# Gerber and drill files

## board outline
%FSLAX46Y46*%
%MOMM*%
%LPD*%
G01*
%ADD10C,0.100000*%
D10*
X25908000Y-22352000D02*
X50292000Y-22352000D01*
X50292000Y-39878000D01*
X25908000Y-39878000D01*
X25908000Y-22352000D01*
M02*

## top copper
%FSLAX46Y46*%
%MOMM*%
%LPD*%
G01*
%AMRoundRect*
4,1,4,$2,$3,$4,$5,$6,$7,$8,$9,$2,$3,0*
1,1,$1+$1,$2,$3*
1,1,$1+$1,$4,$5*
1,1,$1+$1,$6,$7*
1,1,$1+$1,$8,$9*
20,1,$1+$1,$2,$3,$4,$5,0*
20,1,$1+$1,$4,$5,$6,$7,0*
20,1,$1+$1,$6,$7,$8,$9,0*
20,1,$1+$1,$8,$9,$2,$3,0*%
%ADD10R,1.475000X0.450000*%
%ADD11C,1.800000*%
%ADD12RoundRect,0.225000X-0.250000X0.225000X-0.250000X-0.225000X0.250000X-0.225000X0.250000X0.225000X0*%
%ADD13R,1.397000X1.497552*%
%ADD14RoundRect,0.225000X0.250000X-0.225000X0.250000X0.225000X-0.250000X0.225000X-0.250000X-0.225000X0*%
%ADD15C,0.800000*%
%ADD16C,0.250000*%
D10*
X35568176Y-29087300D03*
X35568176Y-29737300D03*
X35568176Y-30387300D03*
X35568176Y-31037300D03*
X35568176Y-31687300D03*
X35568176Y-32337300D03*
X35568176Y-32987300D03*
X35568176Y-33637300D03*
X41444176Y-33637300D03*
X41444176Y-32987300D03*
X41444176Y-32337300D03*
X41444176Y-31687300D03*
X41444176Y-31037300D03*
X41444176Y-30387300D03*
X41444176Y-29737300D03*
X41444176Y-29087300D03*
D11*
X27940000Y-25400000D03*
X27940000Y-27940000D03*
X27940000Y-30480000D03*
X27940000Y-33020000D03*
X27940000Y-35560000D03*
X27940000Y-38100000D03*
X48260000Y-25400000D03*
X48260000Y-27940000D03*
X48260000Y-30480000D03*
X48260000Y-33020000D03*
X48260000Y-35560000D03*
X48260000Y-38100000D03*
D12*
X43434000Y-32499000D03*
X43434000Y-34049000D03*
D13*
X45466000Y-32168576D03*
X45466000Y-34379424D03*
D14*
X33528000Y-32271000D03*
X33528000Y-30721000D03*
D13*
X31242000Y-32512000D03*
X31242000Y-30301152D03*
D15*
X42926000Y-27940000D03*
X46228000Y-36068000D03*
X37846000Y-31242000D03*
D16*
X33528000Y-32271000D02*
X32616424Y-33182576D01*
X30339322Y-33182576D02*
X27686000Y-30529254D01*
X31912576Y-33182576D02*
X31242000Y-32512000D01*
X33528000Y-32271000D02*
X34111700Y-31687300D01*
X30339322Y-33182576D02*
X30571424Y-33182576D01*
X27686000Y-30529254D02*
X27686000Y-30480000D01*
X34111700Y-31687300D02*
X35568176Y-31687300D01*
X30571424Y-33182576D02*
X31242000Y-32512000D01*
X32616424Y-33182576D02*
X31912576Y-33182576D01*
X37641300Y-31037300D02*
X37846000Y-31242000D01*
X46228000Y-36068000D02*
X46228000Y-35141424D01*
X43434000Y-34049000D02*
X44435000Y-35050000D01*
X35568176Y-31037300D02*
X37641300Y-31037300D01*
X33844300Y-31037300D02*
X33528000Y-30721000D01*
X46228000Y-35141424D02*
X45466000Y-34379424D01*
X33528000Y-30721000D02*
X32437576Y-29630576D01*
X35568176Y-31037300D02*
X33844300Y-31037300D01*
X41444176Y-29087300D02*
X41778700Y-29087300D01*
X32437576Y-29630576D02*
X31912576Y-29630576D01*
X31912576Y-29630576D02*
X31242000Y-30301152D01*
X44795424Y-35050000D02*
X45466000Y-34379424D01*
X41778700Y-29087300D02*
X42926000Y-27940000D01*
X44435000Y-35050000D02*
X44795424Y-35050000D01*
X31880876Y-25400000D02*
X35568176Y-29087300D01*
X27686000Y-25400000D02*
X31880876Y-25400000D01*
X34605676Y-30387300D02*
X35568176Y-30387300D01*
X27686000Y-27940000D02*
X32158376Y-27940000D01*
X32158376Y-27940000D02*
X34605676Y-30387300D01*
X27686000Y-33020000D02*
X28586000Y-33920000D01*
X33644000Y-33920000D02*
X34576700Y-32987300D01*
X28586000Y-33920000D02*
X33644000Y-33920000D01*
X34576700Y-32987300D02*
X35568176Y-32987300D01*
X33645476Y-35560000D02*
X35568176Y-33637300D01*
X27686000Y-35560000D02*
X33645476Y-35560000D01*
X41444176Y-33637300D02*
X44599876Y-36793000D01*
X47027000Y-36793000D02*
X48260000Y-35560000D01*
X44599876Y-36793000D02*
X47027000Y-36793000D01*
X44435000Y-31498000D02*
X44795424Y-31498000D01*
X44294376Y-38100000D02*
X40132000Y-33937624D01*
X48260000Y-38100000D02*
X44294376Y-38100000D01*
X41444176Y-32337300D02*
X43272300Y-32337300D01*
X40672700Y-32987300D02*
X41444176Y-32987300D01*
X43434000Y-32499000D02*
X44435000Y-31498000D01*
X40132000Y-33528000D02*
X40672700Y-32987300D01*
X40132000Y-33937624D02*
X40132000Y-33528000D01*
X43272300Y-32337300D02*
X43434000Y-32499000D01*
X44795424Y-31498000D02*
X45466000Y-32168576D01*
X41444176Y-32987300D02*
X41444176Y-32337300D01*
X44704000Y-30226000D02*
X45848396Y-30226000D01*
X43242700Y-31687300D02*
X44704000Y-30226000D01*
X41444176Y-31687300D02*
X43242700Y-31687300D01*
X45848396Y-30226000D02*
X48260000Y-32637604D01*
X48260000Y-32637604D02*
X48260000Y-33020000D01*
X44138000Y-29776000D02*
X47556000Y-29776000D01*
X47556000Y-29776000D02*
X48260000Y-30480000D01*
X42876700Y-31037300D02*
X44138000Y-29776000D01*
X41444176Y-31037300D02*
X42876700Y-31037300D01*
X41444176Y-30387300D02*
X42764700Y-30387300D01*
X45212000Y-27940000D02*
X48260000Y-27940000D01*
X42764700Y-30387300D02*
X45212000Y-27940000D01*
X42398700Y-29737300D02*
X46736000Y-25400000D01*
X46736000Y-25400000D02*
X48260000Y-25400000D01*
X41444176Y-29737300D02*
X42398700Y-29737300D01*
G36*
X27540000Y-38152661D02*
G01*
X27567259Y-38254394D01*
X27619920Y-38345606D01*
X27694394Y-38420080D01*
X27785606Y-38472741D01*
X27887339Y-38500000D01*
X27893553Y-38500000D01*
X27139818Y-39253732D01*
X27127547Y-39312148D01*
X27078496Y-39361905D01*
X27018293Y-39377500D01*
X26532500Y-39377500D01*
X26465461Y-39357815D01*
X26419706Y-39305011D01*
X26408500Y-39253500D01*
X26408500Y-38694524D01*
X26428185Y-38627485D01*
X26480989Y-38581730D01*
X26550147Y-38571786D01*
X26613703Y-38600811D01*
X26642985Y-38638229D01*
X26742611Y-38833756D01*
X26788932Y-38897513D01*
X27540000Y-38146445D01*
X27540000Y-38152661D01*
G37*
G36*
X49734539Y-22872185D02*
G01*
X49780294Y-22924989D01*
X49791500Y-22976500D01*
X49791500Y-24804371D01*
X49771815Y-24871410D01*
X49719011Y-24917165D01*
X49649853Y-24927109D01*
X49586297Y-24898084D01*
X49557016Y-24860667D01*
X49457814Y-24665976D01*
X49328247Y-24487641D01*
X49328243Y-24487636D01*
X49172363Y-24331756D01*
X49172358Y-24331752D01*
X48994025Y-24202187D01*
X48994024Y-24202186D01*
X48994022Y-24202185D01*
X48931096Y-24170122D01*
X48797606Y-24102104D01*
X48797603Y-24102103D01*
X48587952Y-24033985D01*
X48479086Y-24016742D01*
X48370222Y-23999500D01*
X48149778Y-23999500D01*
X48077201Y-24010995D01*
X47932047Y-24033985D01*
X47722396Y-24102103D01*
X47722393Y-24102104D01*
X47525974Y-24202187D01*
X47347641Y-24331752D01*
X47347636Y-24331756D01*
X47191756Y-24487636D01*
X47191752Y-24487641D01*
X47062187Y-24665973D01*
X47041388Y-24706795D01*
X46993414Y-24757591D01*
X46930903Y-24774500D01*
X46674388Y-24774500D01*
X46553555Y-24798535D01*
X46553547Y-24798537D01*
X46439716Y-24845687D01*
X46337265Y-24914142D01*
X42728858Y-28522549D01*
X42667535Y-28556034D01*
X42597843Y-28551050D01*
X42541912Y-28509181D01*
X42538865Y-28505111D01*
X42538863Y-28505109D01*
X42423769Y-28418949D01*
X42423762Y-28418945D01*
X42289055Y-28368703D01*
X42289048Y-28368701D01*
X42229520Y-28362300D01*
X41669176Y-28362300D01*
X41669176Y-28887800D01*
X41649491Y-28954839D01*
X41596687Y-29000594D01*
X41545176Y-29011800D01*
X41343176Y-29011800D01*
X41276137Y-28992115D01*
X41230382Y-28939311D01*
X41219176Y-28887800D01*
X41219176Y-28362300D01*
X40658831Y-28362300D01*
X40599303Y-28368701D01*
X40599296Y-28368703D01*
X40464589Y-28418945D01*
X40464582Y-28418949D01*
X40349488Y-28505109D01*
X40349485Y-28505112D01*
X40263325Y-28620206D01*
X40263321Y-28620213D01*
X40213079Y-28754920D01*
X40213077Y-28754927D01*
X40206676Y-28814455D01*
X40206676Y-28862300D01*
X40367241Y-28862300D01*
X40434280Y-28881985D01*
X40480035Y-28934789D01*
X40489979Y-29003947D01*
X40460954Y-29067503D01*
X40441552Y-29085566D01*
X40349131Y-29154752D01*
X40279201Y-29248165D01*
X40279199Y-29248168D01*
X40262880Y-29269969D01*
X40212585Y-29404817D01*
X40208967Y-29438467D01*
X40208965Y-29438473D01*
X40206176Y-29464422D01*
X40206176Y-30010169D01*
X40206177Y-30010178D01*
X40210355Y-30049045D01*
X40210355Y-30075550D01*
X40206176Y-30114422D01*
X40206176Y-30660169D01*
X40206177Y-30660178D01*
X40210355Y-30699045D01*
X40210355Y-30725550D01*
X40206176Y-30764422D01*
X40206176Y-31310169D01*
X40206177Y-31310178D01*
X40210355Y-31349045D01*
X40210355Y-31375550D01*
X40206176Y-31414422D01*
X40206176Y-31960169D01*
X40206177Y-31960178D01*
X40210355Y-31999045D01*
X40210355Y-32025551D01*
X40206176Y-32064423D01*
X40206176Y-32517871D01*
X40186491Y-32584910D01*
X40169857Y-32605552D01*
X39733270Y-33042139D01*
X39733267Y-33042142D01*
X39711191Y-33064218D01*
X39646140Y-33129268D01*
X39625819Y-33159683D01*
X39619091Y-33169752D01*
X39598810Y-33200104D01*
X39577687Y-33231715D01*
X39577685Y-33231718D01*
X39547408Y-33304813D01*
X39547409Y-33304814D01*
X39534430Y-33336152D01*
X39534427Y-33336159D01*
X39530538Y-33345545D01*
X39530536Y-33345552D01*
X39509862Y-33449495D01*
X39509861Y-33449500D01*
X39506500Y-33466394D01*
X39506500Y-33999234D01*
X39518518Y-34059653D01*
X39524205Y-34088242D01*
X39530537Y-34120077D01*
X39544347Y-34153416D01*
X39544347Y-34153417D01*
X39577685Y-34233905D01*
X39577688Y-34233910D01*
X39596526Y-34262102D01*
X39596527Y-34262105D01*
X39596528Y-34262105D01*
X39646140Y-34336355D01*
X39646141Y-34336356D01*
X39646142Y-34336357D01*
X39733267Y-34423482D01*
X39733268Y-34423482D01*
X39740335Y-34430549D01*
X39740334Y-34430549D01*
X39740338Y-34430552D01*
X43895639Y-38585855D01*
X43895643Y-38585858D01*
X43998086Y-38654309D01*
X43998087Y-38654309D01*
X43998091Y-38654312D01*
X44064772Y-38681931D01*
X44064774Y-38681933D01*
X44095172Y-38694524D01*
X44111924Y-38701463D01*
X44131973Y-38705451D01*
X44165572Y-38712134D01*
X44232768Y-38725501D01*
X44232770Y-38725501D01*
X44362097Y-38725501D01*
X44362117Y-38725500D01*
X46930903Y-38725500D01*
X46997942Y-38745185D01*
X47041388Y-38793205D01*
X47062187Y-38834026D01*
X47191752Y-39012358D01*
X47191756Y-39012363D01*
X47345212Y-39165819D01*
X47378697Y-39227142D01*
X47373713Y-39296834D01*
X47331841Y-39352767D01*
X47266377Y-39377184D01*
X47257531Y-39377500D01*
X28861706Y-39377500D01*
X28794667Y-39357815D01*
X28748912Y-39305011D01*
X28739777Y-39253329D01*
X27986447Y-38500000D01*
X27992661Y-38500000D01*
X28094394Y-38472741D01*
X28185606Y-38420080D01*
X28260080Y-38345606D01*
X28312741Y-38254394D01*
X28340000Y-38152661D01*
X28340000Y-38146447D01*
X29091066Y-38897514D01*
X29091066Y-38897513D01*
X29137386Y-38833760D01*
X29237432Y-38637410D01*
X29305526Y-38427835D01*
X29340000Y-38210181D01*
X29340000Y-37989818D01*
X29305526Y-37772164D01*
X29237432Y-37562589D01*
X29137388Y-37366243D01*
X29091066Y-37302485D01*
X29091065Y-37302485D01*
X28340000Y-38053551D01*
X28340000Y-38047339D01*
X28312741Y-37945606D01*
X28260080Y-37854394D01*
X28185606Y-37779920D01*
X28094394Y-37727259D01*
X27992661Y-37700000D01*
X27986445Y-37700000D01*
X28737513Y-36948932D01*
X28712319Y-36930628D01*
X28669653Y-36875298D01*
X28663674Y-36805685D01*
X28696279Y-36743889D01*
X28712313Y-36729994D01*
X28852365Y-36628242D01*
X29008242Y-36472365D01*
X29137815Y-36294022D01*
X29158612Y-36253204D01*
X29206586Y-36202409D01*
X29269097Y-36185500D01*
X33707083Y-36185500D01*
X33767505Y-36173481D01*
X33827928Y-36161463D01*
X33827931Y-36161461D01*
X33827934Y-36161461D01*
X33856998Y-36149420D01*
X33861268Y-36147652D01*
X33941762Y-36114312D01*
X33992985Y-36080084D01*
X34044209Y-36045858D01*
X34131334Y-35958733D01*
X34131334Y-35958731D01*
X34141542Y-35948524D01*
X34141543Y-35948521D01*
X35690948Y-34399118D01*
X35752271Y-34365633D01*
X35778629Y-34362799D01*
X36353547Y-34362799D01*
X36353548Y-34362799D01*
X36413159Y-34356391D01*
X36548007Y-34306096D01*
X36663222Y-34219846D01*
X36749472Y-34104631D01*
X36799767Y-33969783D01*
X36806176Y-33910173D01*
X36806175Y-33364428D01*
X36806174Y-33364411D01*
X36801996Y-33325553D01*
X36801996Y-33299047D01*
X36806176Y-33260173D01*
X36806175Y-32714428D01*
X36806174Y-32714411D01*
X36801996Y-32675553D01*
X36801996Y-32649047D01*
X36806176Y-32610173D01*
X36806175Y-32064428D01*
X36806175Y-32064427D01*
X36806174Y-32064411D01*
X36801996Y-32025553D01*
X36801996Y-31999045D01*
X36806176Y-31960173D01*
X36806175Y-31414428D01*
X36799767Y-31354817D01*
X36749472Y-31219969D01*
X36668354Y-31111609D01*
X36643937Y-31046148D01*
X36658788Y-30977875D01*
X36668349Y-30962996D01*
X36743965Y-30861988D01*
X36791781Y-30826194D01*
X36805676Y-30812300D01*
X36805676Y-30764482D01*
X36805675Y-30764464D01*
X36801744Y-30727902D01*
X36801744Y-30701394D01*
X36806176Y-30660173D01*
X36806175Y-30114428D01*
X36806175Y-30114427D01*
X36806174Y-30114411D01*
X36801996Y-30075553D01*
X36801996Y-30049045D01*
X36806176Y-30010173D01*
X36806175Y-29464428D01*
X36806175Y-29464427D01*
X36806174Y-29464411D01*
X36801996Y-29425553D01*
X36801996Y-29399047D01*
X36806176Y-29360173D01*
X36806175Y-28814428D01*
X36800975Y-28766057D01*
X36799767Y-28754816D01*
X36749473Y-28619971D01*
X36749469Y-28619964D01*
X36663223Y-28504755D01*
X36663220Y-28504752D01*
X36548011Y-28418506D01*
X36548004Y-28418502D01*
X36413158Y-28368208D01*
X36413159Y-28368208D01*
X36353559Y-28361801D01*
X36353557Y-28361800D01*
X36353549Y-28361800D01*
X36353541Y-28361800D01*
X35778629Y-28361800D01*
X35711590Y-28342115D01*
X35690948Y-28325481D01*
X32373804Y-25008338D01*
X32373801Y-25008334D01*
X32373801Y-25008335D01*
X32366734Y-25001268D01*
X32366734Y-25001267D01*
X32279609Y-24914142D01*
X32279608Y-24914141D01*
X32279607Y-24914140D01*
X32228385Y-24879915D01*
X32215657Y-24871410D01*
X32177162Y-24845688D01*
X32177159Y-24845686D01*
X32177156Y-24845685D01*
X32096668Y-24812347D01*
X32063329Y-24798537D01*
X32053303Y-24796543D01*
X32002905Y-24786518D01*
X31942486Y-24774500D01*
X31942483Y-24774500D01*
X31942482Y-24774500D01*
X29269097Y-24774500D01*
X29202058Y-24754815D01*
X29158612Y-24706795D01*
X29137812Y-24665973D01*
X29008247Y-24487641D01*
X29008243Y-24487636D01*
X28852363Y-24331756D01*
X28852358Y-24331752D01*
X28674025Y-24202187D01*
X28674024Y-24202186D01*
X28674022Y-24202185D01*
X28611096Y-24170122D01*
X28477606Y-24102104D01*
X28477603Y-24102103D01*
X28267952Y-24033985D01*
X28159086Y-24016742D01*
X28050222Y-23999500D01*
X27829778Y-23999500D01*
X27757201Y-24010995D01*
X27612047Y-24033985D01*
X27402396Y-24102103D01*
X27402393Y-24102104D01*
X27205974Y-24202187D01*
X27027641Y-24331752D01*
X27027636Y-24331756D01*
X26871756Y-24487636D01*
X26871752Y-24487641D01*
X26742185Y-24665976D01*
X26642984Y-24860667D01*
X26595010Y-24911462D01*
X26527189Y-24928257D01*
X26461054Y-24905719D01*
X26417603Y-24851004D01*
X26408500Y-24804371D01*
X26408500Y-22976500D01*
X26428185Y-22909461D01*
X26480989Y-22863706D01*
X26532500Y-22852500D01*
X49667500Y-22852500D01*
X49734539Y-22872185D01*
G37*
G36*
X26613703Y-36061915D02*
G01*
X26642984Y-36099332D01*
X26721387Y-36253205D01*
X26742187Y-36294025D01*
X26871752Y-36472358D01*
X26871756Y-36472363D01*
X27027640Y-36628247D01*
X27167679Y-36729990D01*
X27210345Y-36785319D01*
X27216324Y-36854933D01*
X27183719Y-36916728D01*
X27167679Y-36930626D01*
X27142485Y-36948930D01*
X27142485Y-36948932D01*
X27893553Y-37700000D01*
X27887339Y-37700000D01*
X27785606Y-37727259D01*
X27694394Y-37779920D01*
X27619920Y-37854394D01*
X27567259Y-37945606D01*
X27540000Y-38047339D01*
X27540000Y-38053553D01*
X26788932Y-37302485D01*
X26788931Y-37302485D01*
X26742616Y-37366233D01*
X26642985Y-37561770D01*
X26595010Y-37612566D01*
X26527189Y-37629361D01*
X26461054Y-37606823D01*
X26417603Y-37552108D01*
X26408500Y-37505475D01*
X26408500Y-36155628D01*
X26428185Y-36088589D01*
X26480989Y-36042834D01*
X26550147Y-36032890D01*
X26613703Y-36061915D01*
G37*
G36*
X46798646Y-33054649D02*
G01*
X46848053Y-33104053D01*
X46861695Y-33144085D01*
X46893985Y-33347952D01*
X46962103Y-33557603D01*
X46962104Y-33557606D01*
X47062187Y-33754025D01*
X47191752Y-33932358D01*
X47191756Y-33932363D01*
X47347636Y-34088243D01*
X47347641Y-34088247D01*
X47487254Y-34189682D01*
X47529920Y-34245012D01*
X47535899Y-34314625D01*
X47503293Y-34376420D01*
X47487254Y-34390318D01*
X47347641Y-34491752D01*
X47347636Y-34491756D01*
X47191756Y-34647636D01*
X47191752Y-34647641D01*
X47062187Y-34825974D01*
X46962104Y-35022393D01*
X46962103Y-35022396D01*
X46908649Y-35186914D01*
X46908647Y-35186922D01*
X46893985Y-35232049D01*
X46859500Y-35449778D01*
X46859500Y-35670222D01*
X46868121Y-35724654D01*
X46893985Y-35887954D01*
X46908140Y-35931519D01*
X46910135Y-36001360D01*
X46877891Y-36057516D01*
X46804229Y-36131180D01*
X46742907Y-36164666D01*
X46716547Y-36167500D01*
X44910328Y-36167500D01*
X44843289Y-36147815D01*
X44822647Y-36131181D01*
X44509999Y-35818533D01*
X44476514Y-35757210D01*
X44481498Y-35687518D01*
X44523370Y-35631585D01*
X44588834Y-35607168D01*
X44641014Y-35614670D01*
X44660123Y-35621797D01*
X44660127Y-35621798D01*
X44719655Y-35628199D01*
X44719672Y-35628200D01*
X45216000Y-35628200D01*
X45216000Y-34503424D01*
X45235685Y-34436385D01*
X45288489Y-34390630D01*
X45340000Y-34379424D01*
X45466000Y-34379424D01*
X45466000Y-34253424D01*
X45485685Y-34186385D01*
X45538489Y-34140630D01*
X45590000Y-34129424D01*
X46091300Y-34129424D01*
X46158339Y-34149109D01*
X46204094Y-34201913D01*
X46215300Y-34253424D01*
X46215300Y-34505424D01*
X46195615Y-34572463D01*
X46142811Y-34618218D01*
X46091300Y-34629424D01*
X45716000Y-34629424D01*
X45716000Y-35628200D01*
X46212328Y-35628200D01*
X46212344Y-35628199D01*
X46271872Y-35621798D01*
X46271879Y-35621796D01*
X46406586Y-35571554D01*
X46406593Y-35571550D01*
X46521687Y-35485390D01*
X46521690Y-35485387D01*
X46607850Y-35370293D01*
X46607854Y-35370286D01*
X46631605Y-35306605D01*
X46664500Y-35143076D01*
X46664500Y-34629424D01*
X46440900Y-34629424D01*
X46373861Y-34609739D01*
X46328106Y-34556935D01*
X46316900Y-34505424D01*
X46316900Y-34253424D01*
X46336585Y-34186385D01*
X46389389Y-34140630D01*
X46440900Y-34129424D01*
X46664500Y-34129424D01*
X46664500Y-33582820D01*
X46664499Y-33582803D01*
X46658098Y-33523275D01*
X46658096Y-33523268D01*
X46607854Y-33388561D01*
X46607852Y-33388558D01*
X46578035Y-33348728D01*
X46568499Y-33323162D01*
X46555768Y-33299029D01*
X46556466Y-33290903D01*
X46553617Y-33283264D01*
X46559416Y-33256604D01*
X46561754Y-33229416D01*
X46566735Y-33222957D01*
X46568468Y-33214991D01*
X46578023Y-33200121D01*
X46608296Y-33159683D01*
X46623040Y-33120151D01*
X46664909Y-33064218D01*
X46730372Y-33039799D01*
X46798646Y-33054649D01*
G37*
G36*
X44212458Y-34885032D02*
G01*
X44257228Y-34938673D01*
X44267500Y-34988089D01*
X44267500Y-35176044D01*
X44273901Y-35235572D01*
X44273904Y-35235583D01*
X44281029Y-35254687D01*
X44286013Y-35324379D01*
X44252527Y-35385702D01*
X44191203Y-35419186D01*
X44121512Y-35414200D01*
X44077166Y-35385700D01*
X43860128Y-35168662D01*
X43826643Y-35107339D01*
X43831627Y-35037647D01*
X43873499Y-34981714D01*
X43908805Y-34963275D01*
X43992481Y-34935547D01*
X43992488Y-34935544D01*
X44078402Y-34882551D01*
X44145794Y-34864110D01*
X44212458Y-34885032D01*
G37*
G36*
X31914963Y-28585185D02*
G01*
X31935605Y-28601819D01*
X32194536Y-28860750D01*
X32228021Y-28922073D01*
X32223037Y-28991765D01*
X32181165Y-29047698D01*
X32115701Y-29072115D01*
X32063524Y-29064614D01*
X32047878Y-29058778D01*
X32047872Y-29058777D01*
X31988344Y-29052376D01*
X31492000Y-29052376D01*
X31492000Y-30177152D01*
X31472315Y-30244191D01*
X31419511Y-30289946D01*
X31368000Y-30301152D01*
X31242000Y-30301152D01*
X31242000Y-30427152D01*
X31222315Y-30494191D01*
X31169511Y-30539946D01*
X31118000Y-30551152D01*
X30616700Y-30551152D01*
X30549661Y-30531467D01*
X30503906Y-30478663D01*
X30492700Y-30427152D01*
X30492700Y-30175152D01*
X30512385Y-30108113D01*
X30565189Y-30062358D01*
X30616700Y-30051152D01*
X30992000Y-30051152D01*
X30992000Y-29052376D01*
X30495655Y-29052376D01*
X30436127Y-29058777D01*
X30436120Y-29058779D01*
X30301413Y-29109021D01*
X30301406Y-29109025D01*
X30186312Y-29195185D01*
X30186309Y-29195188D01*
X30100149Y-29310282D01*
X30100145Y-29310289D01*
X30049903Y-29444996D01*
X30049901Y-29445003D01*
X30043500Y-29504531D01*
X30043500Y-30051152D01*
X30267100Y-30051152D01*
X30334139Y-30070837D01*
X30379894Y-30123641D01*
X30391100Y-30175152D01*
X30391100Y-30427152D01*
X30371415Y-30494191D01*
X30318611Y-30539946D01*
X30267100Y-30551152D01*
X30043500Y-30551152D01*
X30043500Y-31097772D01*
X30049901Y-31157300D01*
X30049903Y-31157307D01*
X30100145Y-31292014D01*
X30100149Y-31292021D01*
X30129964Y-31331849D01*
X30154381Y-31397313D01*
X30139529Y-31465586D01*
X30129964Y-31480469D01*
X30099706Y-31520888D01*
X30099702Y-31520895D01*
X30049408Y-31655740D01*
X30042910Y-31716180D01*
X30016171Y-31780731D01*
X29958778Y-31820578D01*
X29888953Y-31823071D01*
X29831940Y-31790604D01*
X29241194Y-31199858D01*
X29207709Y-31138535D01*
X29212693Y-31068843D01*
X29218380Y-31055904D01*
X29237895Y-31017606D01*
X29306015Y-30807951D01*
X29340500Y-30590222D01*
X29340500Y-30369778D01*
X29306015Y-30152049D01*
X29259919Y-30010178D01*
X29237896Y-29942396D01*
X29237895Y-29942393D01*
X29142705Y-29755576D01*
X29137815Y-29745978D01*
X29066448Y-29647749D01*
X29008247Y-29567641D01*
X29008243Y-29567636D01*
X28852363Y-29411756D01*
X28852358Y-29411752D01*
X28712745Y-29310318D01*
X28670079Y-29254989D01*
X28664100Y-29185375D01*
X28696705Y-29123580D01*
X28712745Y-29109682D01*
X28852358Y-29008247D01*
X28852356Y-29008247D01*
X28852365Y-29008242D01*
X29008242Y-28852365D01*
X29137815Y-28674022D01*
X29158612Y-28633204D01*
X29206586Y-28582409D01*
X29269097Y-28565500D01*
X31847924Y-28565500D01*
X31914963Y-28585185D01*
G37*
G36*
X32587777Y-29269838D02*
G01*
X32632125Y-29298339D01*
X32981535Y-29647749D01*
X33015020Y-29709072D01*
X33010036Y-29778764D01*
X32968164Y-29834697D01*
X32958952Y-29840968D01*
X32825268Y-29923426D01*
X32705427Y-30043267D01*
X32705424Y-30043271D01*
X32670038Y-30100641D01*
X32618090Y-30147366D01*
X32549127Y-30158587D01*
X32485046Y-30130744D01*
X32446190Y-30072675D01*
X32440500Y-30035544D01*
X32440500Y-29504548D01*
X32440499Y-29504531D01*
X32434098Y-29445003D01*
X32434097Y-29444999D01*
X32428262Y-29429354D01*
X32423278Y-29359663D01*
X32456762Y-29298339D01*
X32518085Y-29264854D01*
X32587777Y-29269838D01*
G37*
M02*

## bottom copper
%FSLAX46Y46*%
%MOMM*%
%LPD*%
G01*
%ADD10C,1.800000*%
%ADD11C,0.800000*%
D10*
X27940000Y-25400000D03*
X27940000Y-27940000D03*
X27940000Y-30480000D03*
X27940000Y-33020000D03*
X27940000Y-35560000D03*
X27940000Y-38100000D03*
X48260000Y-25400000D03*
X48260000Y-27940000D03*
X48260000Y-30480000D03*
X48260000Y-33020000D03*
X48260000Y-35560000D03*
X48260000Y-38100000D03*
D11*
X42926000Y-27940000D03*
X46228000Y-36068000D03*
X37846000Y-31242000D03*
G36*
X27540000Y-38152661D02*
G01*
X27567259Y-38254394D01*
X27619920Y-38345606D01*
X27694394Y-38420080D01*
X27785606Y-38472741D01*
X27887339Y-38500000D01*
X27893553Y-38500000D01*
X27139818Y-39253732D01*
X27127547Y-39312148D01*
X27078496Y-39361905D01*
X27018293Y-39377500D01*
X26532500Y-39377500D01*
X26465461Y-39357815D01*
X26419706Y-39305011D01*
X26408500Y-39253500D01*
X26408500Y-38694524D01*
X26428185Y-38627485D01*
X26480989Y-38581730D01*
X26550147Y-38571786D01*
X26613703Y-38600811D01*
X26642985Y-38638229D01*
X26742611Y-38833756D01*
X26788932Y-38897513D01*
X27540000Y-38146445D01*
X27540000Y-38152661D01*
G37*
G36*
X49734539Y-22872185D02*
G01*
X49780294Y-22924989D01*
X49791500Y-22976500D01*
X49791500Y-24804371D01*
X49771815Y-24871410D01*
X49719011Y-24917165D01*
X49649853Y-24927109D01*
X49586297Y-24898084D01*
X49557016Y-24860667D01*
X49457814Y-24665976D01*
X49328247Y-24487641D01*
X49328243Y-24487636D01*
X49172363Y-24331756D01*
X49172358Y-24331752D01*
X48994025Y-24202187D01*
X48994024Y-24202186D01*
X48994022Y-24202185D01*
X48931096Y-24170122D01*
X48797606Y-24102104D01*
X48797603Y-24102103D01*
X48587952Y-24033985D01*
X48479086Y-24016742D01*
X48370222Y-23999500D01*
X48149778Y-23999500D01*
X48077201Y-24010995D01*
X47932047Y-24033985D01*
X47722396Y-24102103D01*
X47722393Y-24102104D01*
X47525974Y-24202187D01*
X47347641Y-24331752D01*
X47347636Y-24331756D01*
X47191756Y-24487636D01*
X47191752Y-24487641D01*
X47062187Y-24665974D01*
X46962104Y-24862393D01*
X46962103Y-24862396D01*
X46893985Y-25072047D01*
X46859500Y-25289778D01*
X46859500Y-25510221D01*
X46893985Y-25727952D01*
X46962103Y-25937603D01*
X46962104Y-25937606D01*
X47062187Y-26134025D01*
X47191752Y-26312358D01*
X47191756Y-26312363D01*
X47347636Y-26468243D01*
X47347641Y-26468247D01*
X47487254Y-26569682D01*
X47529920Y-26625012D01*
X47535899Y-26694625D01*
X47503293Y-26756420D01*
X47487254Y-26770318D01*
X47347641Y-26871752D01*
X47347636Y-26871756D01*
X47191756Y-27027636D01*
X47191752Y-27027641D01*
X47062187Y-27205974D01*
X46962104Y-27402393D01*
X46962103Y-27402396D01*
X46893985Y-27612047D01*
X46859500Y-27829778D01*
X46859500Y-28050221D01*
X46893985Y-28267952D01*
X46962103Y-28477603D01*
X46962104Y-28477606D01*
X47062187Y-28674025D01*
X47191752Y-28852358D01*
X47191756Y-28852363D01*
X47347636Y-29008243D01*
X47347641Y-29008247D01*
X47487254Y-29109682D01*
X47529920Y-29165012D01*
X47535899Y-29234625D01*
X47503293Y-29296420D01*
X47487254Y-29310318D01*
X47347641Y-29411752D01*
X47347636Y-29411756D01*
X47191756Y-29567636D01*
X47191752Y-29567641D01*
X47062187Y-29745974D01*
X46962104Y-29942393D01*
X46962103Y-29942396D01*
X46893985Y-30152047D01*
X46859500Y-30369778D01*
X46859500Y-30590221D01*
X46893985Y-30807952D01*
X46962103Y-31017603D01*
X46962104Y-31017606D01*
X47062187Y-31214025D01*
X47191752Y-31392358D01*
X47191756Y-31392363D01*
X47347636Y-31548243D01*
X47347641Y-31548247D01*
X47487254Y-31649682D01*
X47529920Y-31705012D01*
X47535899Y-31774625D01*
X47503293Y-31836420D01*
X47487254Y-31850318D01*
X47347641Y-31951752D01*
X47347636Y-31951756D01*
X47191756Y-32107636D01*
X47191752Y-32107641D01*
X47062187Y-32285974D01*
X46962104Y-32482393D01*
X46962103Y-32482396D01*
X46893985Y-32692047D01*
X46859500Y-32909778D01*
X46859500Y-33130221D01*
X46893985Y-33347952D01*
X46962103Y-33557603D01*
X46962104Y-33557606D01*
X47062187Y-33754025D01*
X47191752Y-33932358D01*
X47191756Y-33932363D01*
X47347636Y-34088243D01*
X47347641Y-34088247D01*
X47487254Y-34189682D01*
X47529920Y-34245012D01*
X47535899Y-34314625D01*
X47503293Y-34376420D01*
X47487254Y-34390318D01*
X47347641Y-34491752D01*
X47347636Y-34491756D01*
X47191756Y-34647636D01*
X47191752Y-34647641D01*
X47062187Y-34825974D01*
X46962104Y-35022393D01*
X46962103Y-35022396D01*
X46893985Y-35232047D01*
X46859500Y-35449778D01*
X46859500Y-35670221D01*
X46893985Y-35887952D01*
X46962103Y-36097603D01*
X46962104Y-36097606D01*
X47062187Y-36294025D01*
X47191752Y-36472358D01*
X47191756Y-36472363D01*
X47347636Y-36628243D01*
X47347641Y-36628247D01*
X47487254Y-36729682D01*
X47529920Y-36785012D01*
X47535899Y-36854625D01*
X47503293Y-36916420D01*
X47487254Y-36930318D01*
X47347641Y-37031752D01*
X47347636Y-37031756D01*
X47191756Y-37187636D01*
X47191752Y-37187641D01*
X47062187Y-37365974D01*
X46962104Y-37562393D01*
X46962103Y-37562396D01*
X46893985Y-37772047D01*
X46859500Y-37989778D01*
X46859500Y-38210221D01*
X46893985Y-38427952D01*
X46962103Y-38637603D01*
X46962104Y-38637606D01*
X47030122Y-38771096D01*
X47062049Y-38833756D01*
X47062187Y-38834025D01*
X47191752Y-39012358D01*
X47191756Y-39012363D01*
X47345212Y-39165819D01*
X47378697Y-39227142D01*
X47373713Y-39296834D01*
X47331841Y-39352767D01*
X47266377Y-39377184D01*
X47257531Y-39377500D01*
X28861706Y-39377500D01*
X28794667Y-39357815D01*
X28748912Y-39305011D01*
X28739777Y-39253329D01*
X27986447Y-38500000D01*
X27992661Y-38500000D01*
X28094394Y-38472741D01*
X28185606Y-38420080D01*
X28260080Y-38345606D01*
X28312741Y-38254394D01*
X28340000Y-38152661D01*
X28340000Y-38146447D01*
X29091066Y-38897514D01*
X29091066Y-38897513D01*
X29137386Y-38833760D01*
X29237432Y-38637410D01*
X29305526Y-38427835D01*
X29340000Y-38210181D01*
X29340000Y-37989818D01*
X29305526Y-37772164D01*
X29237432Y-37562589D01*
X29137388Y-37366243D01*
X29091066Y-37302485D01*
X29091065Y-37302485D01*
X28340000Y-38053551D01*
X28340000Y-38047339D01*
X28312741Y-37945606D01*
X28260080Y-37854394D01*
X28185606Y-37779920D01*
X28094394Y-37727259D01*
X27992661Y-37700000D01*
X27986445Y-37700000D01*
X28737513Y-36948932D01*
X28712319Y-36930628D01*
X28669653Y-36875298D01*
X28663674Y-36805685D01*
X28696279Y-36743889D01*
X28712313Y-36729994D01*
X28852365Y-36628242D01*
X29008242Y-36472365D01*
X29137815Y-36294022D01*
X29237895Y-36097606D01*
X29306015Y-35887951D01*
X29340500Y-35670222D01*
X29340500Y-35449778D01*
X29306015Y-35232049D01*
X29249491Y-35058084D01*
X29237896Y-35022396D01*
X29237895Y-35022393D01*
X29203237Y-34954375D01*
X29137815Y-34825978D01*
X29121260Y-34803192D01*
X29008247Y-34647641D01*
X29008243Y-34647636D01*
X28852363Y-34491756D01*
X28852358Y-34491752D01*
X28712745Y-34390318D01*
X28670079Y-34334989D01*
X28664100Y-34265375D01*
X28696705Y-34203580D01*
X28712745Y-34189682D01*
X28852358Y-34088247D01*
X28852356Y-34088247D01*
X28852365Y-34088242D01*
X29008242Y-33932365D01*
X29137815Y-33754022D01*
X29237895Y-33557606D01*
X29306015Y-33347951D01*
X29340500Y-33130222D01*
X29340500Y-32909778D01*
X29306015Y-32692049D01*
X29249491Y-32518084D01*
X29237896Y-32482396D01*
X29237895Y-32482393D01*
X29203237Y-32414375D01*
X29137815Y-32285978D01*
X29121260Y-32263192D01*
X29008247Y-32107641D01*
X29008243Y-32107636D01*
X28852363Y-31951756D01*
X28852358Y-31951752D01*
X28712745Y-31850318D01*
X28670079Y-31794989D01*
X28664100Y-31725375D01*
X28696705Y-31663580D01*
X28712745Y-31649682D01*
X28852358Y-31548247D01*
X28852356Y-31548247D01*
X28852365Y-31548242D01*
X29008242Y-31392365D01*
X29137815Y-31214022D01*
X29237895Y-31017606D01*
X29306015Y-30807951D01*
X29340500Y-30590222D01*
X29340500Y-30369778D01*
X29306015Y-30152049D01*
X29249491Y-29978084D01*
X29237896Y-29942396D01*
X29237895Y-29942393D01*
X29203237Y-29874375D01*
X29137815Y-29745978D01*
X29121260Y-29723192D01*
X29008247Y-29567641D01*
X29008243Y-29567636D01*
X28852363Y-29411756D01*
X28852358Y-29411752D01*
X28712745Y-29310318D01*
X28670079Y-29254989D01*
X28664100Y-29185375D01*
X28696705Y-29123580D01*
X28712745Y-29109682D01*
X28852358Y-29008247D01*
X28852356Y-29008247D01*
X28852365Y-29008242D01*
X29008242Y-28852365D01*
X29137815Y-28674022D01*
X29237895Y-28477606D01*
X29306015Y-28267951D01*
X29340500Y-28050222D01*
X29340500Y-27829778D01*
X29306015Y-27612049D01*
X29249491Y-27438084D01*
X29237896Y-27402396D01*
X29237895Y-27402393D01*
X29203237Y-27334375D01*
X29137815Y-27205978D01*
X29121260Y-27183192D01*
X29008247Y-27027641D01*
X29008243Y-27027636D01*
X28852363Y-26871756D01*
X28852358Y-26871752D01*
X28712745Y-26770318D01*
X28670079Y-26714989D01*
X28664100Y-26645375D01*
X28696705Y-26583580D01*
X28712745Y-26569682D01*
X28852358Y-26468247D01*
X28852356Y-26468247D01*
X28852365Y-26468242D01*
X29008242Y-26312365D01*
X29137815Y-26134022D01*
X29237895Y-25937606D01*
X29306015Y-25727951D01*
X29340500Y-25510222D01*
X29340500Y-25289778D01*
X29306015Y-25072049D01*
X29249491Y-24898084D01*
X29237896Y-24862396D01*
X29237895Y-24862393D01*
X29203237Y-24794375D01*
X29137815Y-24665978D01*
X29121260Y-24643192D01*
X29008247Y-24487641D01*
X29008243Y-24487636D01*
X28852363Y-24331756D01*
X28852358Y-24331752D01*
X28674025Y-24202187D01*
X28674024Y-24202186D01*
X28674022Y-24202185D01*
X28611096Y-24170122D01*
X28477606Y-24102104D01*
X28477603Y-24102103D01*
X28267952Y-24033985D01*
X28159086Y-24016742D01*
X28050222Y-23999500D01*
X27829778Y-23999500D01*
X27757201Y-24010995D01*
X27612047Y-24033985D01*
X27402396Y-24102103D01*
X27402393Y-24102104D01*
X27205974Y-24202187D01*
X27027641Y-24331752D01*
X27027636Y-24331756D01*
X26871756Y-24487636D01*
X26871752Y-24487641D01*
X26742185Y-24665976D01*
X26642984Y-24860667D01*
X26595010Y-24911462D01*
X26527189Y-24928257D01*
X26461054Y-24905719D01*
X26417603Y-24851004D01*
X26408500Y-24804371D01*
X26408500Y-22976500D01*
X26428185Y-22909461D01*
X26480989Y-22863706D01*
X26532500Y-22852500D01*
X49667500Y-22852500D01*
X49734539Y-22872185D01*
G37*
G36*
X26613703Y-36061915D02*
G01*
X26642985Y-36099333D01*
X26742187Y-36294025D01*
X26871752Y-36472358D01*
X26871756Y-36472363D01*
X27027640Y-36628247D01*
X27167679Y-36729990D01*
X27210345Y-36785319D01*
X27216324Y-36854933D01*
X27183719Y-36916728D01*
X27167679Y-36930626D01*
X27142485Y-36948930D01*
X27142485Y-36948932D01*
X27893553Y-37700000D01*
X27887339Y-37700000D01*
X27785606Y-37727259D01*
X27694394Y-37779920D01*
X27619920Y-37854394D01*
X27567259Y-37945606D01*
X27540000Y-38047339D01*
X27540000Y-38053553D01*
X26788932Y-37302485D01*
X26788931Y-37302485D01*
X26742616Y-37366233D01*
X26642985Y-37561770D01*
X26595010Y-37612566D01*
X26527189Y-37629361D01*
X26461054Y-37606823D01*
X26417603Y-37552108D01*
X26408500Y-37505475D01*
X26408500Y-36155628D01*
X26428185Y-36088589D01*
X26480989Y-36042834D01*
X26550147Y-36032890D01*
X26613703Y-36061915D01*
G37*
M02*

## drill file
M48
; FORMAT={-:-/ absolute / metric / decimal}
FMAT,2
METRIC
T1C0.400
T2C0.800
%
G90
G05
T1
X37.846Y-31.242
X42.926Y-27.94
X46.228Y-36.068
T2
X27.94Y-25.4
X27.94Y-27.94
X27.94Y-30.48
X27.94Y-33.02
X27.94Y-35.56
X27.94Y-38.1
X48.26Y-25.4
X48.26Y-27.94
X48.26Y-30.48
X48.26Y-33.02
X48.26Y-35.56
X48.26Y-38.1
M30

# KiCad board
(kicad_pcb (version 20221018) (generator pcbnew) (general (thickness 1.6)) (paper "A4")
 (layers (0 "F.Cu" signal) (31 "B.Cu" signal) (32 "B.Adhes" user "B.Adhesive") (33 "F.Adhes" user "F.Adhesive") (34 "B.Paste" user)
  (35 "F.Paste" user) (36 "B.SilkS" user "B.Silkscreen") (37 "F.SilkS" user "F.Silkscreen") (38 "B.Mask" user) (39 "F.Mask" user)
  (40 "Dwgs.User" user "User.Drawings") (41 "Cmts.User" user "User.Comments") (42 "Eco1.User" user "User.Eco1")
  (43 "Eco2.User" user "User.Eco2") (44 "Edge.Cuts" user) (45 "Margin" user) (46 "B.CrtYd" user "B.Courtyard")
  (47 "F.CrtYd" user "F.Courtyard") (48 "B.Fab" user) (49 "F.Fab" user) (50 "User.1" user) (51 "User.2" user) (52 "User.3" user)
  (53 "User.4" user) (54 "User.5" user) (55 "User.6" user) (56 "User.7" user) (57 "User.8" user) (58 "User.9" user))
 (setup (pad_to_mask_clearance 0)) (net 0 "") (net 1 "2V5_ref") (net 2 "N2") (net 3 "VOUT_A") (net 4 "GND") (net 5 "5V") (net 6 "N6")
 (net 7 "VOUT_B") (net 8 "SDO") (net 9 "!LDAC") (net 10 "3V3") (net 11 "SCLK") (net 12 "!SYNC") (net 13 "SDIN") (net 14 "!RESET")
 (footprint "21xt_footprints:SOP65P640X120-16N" (layer "F.Cu") (at 38.506176 31.3623)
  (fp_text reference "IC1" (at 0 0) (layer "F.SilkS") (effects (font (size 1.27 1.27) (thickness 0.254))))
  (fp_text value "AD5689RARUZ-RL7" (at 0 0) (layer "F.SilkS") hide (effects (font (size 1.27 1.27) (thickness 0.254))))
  (pad "1" smd rect (at -2.938 -2.275 90) (size 0.45 1.475) (layers "F.Cu" "F.Paste" "F.Mask") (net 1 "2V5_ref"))
  (pad "2" smd rect (at -2.938 -1.625 90) (size 0.45 1.475) (layers "F.Cu" "F.Paste" "F.Mask") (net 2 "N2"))
  (pad "3" smd rect (at -2.938 -0.975 90) (size 0.45 1.475) (layers "F.Cu" "F.Paste" "F.Mask") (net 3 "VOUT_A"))
  (pad "4" smd rect (at -2.938 -0.325 90) (size 0.45 1.475) (layers "F.Cu" "F.Paste" "F.Mask") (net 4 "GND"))
  (pad "5" smd rect (at -2.938 0.325 90) (size 0.45 1.475) (layers "F.Cu" "F.Paste" "F.Mask") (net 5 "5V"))
  (pad "6" smd rect (at -2.938 0.975 90) (size 0.45 1.475) (layers "F.Cu" "F.Paste" "F.Mask") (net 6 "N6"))
  (pad "7" smd rect (at -2.938 1.625 90) (size 0.45 1.475) (layers "F.Cu" "F.Paste" "F.Mask") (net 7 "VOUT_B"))
  (pad "8" smd rect (at -2.938 2.275 90) (size 0.45 1.475) (layers "F.Cu" "F.Paste" "F.Mask") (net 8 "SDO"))
  (pad "9" smd rect (at 2.938 2.275 90) (size 0.45 1.475) (layers "F.Cu" "F.Paste" "F.Mask") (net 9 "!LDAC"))
  (pad "10" smd rect (at 2.938 1.625 90) (size 0.45 1.475) (layers "F.Cu" "F.Paste" "F.Mask") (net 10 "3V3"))
  (pad "11" smd rect (at 2.938 0.975 90) (size 0.45 1.475) (layers "F.Cu" "F.Paste" "F.Mask") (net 10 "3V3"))
  (pad "12" smd rect (at 2.938 0.325 90) (size 0.45 1.475) (layers "F.Cu" "F.Paste" "F.Mask") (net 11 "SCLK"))
  (pad "13" smd rect (at 2.938 -0.325 90) (size 0.45 1.475) (layers "F.Cu" "F.Paste" "F.Mask") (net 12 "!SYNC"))
  (pad "14" smd rect (at 2.938 -0.975 90) (size 0.45 1.475) (layers "F.Cu" "F.Paste" "F.Mask") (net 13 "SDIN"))
  (pad "15" smd rect (at 2.938 -1.625 90) (size 0.45 1.475) (layers "F.Cu" "F.Paste" "F.Mask") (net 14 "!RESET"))
  (pad "16" smd rect (at 2.938 -2.275 90) (size 0.45 1.475) (layers "F.Cu" "F.Paste" "F.Mask") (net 4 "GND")))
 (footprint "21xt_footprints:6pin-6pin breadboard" (layer "F.Cu") (at 35.56 38.1)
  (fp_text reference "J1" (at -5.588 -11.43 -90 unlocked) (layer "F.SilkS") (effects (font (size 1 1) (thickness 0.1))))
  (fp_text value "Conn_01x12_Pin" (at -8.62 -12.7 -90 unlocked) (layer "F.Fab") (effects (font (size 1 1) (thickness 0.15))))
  (pad "1" thru_hole circle (at -7.62 -12.7 270) (size 1.8 1.8) (drill 0.8) (layers "*.Cu" "*.Mask") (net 1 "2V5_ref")
   (solder_mask_margin 0.102))
  (pad "2" thru_hole circle (at -7.62 -10.16 270) (size 1.8 1.8) (drill 0.8) (layers "*.Cu" "*.Mask") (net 3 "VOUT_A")
   (solder_mask_margin 0.102))
  (pad "3" thru_hole circle (at -7.62 -7.62 270) (size 1.8 1.8) (drill 0.8) (layers "*.Cu" "*.Mask") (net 5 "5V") (solder_mask_margin 0.102))
  (pad "4" thru_hole circle (at -7.62 -5.08 270) (size 1.8 1.8) (drill 0.8) (layers "*.Cu" "*.Mask") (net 7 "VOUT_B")
   (solder_mask_margin 0.102))
  (pad "5" thru_hole circle (at -7.62 -2.54 270) (size 1.8 1.8) (drill 0.8) (layers "*.Cu" "*.Mask") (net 8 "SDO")
   (solder_mask_margin 0.102))
  (pad "6" thru_hole circle (at -7.62 0 270) (size 1.8 1.8) (drill 0.8) (layers "*.Cu" "*.Mask") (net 4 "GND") (solder_mask_margin 0.102))
  (pad "7" thru_hole circle (at 12.7 -12.7 270) (size 1.8 1.8) (drill 0.8) (layers "*.Cu" "*.Mask") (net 14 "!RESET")
   (solder_mask_margin 0.102))
  (pad "8" thru_hole circle (at 12.7 -10.16 270) (size 1.8 1.8) (drill 0.8) (layers "*.Cu" "*.Mask") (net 13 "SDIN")
   (solder_mask_margin 0.102))
  (pad "9" thru_hole circle (at 12.7 -7.62 270) (size 1.8 1.8) (drill 0.8) (layers "*.Cu" "*.Mask") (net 12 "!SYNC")
   (solder_mask_margin 0.102))
  (pad "10" thru_hole circle (at 12.7 -5.08 270) (size 1.8 1.8) (drill 0.8) (layers "*.Cu" "*.Mask") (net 11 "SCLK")
   (solder_mask_margin 0.102))
  (pad "11" thru_hole circle (at 12.7 -2.54 270) (size 1.8 1.8) (drill 0.8) (layers "*.Cu" "*.Mask") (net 9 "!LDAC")
   (solder_mask_margin 0.102))
  (pad "12" thru_hole circle (at 12.7 0 270) (size 1.8 1.8) (drill 0.8) (layers "*.Cu" "*.Mask") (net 10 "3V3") (solder_mask_margin 0.102)))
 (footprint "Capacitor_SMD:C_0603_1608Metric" (layer "F.Cu") (at 43.434 33.274 -90)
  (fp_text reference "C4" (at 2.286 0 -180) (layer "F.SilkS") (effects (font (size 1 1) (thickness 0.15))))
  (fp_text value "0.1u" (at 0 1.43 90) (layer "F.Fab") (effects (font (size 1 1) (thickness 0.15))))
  (pad "1" smd roundrect (at -0.775 0 270) (size 0.9 0.95) (layers "F.Cu" "F.Paste" "F.Mask") (roundrect_rratio 0.25) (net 10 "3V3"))
  (pad "2" smd roundrect (at 0.775 0 270) (size 0.9 0.95) (layers "F.Cu" "F.Paste" "F.Mask") (roundrect_rratio 0.25) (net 4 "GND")))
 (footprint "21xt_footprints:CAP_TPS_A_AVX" (layer "F.Cu") (at 45.466 33.274 -90)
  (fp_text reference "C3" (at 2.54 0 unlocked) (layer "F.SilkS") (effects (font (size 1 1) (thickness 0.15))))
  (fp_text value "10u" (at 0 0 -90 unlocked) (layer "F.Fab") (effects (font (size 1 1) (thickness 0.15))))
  (pad "1" smd rect (at -1.105424 0) (size 1.397 1.497552) (layers "F.Cu" "F.Paste" "F.Mask") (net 10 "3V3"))
  (pad "2" smd rect (at 1.105424 0) (size 1.397 1.497552) (layers "F.Cu" "F.Paste" "F.Mask") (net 4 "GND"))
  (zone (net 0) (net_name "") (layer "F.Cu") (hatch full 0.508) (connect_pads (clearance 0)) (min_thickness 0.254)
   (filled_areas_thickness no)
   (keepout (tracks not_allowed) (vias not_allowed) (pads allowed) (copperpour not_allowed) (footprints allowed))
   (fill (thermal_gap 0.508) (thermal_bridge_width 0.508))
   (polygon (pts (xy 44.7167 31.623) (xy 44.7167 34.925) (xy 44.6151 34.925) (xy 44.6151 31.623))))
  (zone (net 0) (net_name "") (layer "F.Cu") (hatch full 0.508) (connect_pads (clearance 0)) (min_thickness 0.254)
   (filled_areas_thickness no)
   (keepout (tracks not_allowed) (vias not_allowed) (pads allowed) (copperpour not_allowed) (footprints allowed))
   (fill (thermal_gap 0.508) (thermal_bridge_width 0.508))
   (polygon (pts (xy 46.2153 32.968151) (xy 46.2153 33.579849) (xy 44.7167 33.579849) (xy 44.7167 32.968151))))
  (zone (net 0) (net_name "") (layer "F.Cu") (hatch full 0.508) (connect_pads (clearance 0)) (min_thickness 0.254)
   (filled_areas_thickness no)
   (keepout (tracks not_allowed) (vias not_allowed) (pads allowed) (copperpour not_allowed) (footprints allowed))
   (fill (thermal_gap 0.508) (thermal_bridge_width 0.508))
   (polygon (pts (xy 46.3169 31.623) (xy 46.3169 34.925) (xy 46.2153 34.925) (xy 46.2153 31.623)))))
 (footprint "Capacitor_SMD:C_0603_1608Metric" (layer "F.Cu") (at 33.528 31.496 90)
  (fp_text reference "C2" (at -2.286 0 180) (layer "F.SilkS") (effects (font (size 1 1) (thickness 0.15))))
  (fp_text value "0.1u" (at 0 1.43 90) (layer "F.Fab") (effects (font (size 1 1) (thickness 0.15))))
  (pad "1" smd roundrect (at -0.775 0 90) (size 0.9 0.95) (layers "F.Cu" "F.Paste" "F.Mask") (roundrect_rratio 0.25) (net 5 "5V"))
  (pad "2" smd roundrect (at 0.775 0 90) (size 0.9 0.95) (layers "F.Cu" "F.Paste" "F.Mask") (roundrect_rratio 0.25) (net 4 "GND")))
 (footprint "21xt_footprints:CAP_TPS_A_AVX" (layer "F.Cu") (at 31.242 31.406576 90)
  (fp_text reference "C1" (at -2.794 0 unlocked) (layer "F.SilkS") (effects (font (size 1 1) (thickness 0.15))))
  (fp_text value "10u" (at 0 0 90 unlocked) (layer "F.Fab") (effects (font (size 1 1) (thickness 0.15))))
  (pad "1" smd rect (at -1.105424 0 180) (size 1.397 1.497552) (layers "F.Cu" "F.Paste" "F.Mask") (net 5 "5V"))
  (pad "2" smd rect (at 1.105424 0 180) (size 1.397 1.497552) (layers "F.Cu" "F.Paste" "F.Mask") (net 4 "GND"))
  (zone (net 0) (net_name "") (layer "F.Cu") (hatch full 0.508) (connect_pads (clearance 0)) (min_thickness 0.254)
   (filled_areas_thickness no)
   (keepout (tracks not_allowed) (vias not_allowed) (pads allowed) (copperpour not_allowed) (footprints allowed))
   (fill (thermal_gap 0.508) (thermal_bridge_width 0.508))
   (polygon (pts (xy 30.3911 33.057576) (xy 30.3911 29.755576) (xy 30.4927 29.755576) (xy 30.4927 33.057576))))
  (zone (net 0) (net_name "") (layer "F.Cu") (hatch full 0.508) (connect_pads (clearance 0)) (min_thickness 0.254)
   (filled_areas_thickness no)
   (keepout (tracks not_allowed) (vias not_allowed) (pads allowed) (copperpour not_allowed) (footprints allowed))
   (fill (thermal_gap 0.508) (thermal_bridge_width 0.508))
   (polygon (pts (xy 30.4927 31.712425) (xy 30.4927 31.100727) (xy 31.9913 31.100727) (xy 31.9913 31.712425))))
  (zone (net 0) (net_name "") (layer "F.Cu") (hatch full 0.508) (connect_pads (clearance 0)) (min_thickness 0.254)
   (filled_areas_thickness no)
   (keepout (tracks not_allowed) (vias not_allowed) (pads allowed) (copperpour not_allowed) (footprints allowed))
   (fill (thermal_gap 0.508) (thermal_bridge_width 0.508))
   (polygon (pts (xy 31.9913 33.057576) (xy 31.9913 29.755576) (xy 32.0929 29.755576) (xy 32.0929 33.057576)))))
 (gr_rect (start 25.908 22.352) (end 50.292 39.878) (stroke (width 0.1) (type default)) (fill none) (layer "Edge.Cuts"))
 (segment (start 33.528 32.271) (end 32.616424 33.182576) (width 0.25) (layer "F.Cu") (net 5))
 (segment (start 30.339322 33.182576) (end 27.686 30.529254) (width 0.25) (layer "F.Cu") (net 5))
 (segment (start 31.912576 33.182576) (end 31.242 32.512) (width 0.25) (layer "F.Cu") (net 5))
 (segment (start 33.528 32.271) (end 34.1117 31.6873) (width 0.25) (layer "F.Cu") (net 5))
 (segment (start 30.339322 33.182576) (end 30.571424 33.182576) (width 0.25) (layer "F.Cu") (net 5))
 (segment (start 27.686 30.529254) (end 27.686 30.48) (width 0.25) (layer "F.Cu") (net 5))
 (segment (start 34.1117 31.6873) (end 35.568176 31.6873) (width 0.25) (layer "F.Cu") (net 5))
 (segment (start 30.571424 33.182576) (end 31.242 32.512) (width 0.25) (layer "F.Cu") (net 5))
 (segment (start 32.616424 33.182576) (end 31.912576 33.182576) (width 0.25) (layer "F.Cu") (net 5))
 (segment (start 37.6413 31.0373) (end 37.846 31.242) (width 0.25) (layer "F.Cu") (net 4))
 (segment (start 46.228 36.068) (end 46.228 35.141424) (width 0.25) (layer "F.Cu") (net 4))
 (segment (start 43.434 34.049) (end 44.435 35.05) (width 0.25) (layer "F.Cu") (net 4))
 (segment (start 35.568176 31.0373) (end 37.6413 31.0373) (width 0.25) (layer "F.Cu") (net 4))
 (segment (start 33.8443 31.0373) (end 33.528 30.721) (width 0.25) (layer "F.Cu") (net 4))
 (segment (start 46.228 35.141424) (end 45.466 34.379424) (width 0.25) (layer "F.Cu") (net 4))
 (segment (start 33.528 30.721) (end 32.437576 29.630576) (width 0.25) (layer "F.Cu") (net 4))
 (segment (start 35.568176 31.0373) (end 33.8443 31.0373) (width 0.25) (layer "F.Cu") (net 4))
 (segment (start 41.444176 29.0873) (end 41.7787 29.0873) (width 0.25) (layer "F.Cu") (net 4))
 (segment (start 32.437576 29.630576) (end 31.912576 29.630576) (width 0.25) (layer "F.Cu") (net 4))
 (segment (start 31.912576 29.630576) (end 31.242 30.301152) (width 0.25) (layer "F.Cu") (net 4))
 (segment (start 44.795424 35.05) (end 45.466 34.379424) (width 0.25) (layer "F.Cu") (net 4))
 (segment (start 41.7787 29.0873) (end 42.926 27.94) (width 0.25) (layer "F.Cu") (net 4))
 (segment (start 44.435 35.05) (end 44.795424 35.05) (width 0.25) (layer "F.Cu") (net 4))
 (via (at 42.926 27.94) (size 0.8) (drill 0.4) (layers "F.Cu" "B.Cu") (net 4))
 (via (at 46.228 36.068) (size 0.8) (drill 0.4) (layers "F.Cu" "B.Cu") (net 4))
 (via (at 37.846 31.242) (size 0.8) (drill 0.4) (layers "F.Cu" "B.Cu") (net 4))
 (segment (start 31.880876 25.4) (end 35.568176 29.0873) (width 0.25) (layer "F.Cu") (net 1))
 (segment (start 27.686 25.4) (end 31.880876 25.4) (width 0.25) (layer "F.Cu") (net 1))
 (segment (start 34.605676 30.3873) (end 35.568176 30.3873) (width 0.25) (layer "F.Cu") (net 3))
 (segment (start 27.686 27.94) (end 32.158376 27.94) (width 0.25) (layer "F.Cu") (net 3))
 (segment (start 32.158376 27.94) (end 34.605676 30.3873) (width 0.25) (layer "F.Cu") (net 3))
 (segment (start 27.686 33.02) (end 28.586 33.92) (width 0.25) (layer "F.Cu") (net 7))
 (segment (start 33.644 33.92) (end 34.5767 32.9873) (width 0.25) (layer "F.Cu") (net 7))
 (segment (start 28.586 33.92) (end 33.644 33.92) (width 0.25) (layer "F.Cu") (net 7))
 (segment (start 34.5767 32.9873) (end 35.568176 32.9873) (width 0.25) (layer "F.Cu") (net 7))
 (segment (start 33.645476 35.56) (end 35.568176 33.6373) (width 0.25) (layer "F.Cu") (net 8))
 (segment (start 27.686 35.56) (end 33.645476 35.56) (width 0.25) (layer "F.Cu") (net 8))
 (segment (start 41.444176 33.6373) (end 44.599876 36.793) (width 0.25) (layer "F.Cu") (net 9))
 (segment (start 47.027 36.793) (end 48.26 35.56) (width 0.25) (layer "F.Cu") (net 9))
 (segment (start 44.599876 36.793) (end 47.027 36.793) (width 0.25) (layer "F.Cu") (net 9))
 (segment (start 44.435 31.498) (end 44.795424 31.498) (width 0.25) (layer "F.Cu") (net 10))
 (segment (start 44.294376 38.1) (end 40.132 33.937624) (width 0.25) (layer "F.Cu") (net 10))
 (segment (start 48.26 38.1) (end 44.294376 38.1) (width 0.25) (layer "F.Cu") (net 10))
 (segment (start 41.444176 32.3373) (end 43.2723 32.3373) (width 0.25) (layer "F.Cu") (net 10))
 (segment (start 40.6727 32.9873) (end 41.444176 32.9873) (width 0.25) (layer "F.Cu") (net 10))
 (segment (start 43.434 32.499) (end 44.435 31.498) (width 0.25) (layer "F.Cu") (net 10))
 (segment (start 40.132 33.528) (end 40.6727 32.9873) (width 0.25) (layer "F.Cu") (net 10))
 (segment (start 40.132 33.937624) (end 40.132 33.528) (width 0.25) (layer "F.Cu") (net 10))
 (segment (start 43.2723 32.3373) (end 43.434 32.499) (width 0.25) (layer "F.Cu") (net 10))
 (segment (start 44.795424 31.498) (end 45.466 32.168576) (width 0.25) (layer "F.Cu") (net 10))
 (segment (start 41.444176 32.9873) (end 41.444176 32.3373) (width 0.25) (layer "F.Cu") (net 10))
 (segment (start 44.704 30.226) (end 45.848396 30.226) (width 0.25) (layer "F.Cu") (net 11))
 (segment (start 43.2427 31.6873) (end 44.704 30.226) (width 0.25) (layer "F.Cu") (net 11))
 (segment (start 41.444176 31.6873) (end 43.2427 31.6873) (width 0.25) (layer "F.Cu") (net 11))
 (segment (start 45.848396 30.226) (end 48.26 32.637604) (width 0.25) (layer "F.Cu") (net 11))
 (segment (start 48.26 32.637604) (end 48.26 33.02) (width 0.25) (layer "F.Cu") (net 11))
 (segment (start 44.138 29.776) (end 47.556 29.776) (width 0.25) (layer "F.Cu") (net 12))
 (segment (start 47.556 29.776) (end 48.26 30.48) (width 0.25) (layer "F.Cu") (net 12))
 (segment (start 42.8767 31.0373) (end 44.138 29.776) (width 0.25) (layer "F.Cu") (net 12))
 (segment (start 41.444176 31.0373) (end 42.8767 31.0373) (width 0.25) (layer "F.Cu") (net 12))
 (segment (start 41.444176 30.3873) (end 42.7647 30.3873) (width 0.25) (layer "F.Cu") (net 13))
 (segment (start 45.212 27.94) (end 48.26 27.94) (width 0.25) (layer "F.Cu") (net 13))
 (segment (start 42.7647 30.3873) (end 45.212 27.94) (width 0.25) (layer "F.Cu") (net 13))
 (segment (start 42.3987 29.7373) (end 46.736 25.4) (width 0.25) (layer "F.Cu") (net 14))
 (segment (start 46.736 25.4) (end 48.26 25.4) (width 0.25) (layer "F.Cu") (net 14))
 (segment (start 41.444176 29.7373) (end 42.3987 29.7373) (width 0.25) (layer "F.Cu") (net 14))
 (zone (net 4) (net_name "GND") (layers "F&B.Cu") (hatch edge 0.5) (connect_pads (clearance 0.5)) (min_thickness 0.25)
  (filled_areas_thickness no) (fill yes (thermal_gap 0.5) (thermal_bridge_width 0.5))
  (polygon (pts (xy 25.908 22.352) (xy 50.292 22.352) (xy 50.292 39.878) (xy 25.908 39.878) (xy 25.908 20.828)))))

